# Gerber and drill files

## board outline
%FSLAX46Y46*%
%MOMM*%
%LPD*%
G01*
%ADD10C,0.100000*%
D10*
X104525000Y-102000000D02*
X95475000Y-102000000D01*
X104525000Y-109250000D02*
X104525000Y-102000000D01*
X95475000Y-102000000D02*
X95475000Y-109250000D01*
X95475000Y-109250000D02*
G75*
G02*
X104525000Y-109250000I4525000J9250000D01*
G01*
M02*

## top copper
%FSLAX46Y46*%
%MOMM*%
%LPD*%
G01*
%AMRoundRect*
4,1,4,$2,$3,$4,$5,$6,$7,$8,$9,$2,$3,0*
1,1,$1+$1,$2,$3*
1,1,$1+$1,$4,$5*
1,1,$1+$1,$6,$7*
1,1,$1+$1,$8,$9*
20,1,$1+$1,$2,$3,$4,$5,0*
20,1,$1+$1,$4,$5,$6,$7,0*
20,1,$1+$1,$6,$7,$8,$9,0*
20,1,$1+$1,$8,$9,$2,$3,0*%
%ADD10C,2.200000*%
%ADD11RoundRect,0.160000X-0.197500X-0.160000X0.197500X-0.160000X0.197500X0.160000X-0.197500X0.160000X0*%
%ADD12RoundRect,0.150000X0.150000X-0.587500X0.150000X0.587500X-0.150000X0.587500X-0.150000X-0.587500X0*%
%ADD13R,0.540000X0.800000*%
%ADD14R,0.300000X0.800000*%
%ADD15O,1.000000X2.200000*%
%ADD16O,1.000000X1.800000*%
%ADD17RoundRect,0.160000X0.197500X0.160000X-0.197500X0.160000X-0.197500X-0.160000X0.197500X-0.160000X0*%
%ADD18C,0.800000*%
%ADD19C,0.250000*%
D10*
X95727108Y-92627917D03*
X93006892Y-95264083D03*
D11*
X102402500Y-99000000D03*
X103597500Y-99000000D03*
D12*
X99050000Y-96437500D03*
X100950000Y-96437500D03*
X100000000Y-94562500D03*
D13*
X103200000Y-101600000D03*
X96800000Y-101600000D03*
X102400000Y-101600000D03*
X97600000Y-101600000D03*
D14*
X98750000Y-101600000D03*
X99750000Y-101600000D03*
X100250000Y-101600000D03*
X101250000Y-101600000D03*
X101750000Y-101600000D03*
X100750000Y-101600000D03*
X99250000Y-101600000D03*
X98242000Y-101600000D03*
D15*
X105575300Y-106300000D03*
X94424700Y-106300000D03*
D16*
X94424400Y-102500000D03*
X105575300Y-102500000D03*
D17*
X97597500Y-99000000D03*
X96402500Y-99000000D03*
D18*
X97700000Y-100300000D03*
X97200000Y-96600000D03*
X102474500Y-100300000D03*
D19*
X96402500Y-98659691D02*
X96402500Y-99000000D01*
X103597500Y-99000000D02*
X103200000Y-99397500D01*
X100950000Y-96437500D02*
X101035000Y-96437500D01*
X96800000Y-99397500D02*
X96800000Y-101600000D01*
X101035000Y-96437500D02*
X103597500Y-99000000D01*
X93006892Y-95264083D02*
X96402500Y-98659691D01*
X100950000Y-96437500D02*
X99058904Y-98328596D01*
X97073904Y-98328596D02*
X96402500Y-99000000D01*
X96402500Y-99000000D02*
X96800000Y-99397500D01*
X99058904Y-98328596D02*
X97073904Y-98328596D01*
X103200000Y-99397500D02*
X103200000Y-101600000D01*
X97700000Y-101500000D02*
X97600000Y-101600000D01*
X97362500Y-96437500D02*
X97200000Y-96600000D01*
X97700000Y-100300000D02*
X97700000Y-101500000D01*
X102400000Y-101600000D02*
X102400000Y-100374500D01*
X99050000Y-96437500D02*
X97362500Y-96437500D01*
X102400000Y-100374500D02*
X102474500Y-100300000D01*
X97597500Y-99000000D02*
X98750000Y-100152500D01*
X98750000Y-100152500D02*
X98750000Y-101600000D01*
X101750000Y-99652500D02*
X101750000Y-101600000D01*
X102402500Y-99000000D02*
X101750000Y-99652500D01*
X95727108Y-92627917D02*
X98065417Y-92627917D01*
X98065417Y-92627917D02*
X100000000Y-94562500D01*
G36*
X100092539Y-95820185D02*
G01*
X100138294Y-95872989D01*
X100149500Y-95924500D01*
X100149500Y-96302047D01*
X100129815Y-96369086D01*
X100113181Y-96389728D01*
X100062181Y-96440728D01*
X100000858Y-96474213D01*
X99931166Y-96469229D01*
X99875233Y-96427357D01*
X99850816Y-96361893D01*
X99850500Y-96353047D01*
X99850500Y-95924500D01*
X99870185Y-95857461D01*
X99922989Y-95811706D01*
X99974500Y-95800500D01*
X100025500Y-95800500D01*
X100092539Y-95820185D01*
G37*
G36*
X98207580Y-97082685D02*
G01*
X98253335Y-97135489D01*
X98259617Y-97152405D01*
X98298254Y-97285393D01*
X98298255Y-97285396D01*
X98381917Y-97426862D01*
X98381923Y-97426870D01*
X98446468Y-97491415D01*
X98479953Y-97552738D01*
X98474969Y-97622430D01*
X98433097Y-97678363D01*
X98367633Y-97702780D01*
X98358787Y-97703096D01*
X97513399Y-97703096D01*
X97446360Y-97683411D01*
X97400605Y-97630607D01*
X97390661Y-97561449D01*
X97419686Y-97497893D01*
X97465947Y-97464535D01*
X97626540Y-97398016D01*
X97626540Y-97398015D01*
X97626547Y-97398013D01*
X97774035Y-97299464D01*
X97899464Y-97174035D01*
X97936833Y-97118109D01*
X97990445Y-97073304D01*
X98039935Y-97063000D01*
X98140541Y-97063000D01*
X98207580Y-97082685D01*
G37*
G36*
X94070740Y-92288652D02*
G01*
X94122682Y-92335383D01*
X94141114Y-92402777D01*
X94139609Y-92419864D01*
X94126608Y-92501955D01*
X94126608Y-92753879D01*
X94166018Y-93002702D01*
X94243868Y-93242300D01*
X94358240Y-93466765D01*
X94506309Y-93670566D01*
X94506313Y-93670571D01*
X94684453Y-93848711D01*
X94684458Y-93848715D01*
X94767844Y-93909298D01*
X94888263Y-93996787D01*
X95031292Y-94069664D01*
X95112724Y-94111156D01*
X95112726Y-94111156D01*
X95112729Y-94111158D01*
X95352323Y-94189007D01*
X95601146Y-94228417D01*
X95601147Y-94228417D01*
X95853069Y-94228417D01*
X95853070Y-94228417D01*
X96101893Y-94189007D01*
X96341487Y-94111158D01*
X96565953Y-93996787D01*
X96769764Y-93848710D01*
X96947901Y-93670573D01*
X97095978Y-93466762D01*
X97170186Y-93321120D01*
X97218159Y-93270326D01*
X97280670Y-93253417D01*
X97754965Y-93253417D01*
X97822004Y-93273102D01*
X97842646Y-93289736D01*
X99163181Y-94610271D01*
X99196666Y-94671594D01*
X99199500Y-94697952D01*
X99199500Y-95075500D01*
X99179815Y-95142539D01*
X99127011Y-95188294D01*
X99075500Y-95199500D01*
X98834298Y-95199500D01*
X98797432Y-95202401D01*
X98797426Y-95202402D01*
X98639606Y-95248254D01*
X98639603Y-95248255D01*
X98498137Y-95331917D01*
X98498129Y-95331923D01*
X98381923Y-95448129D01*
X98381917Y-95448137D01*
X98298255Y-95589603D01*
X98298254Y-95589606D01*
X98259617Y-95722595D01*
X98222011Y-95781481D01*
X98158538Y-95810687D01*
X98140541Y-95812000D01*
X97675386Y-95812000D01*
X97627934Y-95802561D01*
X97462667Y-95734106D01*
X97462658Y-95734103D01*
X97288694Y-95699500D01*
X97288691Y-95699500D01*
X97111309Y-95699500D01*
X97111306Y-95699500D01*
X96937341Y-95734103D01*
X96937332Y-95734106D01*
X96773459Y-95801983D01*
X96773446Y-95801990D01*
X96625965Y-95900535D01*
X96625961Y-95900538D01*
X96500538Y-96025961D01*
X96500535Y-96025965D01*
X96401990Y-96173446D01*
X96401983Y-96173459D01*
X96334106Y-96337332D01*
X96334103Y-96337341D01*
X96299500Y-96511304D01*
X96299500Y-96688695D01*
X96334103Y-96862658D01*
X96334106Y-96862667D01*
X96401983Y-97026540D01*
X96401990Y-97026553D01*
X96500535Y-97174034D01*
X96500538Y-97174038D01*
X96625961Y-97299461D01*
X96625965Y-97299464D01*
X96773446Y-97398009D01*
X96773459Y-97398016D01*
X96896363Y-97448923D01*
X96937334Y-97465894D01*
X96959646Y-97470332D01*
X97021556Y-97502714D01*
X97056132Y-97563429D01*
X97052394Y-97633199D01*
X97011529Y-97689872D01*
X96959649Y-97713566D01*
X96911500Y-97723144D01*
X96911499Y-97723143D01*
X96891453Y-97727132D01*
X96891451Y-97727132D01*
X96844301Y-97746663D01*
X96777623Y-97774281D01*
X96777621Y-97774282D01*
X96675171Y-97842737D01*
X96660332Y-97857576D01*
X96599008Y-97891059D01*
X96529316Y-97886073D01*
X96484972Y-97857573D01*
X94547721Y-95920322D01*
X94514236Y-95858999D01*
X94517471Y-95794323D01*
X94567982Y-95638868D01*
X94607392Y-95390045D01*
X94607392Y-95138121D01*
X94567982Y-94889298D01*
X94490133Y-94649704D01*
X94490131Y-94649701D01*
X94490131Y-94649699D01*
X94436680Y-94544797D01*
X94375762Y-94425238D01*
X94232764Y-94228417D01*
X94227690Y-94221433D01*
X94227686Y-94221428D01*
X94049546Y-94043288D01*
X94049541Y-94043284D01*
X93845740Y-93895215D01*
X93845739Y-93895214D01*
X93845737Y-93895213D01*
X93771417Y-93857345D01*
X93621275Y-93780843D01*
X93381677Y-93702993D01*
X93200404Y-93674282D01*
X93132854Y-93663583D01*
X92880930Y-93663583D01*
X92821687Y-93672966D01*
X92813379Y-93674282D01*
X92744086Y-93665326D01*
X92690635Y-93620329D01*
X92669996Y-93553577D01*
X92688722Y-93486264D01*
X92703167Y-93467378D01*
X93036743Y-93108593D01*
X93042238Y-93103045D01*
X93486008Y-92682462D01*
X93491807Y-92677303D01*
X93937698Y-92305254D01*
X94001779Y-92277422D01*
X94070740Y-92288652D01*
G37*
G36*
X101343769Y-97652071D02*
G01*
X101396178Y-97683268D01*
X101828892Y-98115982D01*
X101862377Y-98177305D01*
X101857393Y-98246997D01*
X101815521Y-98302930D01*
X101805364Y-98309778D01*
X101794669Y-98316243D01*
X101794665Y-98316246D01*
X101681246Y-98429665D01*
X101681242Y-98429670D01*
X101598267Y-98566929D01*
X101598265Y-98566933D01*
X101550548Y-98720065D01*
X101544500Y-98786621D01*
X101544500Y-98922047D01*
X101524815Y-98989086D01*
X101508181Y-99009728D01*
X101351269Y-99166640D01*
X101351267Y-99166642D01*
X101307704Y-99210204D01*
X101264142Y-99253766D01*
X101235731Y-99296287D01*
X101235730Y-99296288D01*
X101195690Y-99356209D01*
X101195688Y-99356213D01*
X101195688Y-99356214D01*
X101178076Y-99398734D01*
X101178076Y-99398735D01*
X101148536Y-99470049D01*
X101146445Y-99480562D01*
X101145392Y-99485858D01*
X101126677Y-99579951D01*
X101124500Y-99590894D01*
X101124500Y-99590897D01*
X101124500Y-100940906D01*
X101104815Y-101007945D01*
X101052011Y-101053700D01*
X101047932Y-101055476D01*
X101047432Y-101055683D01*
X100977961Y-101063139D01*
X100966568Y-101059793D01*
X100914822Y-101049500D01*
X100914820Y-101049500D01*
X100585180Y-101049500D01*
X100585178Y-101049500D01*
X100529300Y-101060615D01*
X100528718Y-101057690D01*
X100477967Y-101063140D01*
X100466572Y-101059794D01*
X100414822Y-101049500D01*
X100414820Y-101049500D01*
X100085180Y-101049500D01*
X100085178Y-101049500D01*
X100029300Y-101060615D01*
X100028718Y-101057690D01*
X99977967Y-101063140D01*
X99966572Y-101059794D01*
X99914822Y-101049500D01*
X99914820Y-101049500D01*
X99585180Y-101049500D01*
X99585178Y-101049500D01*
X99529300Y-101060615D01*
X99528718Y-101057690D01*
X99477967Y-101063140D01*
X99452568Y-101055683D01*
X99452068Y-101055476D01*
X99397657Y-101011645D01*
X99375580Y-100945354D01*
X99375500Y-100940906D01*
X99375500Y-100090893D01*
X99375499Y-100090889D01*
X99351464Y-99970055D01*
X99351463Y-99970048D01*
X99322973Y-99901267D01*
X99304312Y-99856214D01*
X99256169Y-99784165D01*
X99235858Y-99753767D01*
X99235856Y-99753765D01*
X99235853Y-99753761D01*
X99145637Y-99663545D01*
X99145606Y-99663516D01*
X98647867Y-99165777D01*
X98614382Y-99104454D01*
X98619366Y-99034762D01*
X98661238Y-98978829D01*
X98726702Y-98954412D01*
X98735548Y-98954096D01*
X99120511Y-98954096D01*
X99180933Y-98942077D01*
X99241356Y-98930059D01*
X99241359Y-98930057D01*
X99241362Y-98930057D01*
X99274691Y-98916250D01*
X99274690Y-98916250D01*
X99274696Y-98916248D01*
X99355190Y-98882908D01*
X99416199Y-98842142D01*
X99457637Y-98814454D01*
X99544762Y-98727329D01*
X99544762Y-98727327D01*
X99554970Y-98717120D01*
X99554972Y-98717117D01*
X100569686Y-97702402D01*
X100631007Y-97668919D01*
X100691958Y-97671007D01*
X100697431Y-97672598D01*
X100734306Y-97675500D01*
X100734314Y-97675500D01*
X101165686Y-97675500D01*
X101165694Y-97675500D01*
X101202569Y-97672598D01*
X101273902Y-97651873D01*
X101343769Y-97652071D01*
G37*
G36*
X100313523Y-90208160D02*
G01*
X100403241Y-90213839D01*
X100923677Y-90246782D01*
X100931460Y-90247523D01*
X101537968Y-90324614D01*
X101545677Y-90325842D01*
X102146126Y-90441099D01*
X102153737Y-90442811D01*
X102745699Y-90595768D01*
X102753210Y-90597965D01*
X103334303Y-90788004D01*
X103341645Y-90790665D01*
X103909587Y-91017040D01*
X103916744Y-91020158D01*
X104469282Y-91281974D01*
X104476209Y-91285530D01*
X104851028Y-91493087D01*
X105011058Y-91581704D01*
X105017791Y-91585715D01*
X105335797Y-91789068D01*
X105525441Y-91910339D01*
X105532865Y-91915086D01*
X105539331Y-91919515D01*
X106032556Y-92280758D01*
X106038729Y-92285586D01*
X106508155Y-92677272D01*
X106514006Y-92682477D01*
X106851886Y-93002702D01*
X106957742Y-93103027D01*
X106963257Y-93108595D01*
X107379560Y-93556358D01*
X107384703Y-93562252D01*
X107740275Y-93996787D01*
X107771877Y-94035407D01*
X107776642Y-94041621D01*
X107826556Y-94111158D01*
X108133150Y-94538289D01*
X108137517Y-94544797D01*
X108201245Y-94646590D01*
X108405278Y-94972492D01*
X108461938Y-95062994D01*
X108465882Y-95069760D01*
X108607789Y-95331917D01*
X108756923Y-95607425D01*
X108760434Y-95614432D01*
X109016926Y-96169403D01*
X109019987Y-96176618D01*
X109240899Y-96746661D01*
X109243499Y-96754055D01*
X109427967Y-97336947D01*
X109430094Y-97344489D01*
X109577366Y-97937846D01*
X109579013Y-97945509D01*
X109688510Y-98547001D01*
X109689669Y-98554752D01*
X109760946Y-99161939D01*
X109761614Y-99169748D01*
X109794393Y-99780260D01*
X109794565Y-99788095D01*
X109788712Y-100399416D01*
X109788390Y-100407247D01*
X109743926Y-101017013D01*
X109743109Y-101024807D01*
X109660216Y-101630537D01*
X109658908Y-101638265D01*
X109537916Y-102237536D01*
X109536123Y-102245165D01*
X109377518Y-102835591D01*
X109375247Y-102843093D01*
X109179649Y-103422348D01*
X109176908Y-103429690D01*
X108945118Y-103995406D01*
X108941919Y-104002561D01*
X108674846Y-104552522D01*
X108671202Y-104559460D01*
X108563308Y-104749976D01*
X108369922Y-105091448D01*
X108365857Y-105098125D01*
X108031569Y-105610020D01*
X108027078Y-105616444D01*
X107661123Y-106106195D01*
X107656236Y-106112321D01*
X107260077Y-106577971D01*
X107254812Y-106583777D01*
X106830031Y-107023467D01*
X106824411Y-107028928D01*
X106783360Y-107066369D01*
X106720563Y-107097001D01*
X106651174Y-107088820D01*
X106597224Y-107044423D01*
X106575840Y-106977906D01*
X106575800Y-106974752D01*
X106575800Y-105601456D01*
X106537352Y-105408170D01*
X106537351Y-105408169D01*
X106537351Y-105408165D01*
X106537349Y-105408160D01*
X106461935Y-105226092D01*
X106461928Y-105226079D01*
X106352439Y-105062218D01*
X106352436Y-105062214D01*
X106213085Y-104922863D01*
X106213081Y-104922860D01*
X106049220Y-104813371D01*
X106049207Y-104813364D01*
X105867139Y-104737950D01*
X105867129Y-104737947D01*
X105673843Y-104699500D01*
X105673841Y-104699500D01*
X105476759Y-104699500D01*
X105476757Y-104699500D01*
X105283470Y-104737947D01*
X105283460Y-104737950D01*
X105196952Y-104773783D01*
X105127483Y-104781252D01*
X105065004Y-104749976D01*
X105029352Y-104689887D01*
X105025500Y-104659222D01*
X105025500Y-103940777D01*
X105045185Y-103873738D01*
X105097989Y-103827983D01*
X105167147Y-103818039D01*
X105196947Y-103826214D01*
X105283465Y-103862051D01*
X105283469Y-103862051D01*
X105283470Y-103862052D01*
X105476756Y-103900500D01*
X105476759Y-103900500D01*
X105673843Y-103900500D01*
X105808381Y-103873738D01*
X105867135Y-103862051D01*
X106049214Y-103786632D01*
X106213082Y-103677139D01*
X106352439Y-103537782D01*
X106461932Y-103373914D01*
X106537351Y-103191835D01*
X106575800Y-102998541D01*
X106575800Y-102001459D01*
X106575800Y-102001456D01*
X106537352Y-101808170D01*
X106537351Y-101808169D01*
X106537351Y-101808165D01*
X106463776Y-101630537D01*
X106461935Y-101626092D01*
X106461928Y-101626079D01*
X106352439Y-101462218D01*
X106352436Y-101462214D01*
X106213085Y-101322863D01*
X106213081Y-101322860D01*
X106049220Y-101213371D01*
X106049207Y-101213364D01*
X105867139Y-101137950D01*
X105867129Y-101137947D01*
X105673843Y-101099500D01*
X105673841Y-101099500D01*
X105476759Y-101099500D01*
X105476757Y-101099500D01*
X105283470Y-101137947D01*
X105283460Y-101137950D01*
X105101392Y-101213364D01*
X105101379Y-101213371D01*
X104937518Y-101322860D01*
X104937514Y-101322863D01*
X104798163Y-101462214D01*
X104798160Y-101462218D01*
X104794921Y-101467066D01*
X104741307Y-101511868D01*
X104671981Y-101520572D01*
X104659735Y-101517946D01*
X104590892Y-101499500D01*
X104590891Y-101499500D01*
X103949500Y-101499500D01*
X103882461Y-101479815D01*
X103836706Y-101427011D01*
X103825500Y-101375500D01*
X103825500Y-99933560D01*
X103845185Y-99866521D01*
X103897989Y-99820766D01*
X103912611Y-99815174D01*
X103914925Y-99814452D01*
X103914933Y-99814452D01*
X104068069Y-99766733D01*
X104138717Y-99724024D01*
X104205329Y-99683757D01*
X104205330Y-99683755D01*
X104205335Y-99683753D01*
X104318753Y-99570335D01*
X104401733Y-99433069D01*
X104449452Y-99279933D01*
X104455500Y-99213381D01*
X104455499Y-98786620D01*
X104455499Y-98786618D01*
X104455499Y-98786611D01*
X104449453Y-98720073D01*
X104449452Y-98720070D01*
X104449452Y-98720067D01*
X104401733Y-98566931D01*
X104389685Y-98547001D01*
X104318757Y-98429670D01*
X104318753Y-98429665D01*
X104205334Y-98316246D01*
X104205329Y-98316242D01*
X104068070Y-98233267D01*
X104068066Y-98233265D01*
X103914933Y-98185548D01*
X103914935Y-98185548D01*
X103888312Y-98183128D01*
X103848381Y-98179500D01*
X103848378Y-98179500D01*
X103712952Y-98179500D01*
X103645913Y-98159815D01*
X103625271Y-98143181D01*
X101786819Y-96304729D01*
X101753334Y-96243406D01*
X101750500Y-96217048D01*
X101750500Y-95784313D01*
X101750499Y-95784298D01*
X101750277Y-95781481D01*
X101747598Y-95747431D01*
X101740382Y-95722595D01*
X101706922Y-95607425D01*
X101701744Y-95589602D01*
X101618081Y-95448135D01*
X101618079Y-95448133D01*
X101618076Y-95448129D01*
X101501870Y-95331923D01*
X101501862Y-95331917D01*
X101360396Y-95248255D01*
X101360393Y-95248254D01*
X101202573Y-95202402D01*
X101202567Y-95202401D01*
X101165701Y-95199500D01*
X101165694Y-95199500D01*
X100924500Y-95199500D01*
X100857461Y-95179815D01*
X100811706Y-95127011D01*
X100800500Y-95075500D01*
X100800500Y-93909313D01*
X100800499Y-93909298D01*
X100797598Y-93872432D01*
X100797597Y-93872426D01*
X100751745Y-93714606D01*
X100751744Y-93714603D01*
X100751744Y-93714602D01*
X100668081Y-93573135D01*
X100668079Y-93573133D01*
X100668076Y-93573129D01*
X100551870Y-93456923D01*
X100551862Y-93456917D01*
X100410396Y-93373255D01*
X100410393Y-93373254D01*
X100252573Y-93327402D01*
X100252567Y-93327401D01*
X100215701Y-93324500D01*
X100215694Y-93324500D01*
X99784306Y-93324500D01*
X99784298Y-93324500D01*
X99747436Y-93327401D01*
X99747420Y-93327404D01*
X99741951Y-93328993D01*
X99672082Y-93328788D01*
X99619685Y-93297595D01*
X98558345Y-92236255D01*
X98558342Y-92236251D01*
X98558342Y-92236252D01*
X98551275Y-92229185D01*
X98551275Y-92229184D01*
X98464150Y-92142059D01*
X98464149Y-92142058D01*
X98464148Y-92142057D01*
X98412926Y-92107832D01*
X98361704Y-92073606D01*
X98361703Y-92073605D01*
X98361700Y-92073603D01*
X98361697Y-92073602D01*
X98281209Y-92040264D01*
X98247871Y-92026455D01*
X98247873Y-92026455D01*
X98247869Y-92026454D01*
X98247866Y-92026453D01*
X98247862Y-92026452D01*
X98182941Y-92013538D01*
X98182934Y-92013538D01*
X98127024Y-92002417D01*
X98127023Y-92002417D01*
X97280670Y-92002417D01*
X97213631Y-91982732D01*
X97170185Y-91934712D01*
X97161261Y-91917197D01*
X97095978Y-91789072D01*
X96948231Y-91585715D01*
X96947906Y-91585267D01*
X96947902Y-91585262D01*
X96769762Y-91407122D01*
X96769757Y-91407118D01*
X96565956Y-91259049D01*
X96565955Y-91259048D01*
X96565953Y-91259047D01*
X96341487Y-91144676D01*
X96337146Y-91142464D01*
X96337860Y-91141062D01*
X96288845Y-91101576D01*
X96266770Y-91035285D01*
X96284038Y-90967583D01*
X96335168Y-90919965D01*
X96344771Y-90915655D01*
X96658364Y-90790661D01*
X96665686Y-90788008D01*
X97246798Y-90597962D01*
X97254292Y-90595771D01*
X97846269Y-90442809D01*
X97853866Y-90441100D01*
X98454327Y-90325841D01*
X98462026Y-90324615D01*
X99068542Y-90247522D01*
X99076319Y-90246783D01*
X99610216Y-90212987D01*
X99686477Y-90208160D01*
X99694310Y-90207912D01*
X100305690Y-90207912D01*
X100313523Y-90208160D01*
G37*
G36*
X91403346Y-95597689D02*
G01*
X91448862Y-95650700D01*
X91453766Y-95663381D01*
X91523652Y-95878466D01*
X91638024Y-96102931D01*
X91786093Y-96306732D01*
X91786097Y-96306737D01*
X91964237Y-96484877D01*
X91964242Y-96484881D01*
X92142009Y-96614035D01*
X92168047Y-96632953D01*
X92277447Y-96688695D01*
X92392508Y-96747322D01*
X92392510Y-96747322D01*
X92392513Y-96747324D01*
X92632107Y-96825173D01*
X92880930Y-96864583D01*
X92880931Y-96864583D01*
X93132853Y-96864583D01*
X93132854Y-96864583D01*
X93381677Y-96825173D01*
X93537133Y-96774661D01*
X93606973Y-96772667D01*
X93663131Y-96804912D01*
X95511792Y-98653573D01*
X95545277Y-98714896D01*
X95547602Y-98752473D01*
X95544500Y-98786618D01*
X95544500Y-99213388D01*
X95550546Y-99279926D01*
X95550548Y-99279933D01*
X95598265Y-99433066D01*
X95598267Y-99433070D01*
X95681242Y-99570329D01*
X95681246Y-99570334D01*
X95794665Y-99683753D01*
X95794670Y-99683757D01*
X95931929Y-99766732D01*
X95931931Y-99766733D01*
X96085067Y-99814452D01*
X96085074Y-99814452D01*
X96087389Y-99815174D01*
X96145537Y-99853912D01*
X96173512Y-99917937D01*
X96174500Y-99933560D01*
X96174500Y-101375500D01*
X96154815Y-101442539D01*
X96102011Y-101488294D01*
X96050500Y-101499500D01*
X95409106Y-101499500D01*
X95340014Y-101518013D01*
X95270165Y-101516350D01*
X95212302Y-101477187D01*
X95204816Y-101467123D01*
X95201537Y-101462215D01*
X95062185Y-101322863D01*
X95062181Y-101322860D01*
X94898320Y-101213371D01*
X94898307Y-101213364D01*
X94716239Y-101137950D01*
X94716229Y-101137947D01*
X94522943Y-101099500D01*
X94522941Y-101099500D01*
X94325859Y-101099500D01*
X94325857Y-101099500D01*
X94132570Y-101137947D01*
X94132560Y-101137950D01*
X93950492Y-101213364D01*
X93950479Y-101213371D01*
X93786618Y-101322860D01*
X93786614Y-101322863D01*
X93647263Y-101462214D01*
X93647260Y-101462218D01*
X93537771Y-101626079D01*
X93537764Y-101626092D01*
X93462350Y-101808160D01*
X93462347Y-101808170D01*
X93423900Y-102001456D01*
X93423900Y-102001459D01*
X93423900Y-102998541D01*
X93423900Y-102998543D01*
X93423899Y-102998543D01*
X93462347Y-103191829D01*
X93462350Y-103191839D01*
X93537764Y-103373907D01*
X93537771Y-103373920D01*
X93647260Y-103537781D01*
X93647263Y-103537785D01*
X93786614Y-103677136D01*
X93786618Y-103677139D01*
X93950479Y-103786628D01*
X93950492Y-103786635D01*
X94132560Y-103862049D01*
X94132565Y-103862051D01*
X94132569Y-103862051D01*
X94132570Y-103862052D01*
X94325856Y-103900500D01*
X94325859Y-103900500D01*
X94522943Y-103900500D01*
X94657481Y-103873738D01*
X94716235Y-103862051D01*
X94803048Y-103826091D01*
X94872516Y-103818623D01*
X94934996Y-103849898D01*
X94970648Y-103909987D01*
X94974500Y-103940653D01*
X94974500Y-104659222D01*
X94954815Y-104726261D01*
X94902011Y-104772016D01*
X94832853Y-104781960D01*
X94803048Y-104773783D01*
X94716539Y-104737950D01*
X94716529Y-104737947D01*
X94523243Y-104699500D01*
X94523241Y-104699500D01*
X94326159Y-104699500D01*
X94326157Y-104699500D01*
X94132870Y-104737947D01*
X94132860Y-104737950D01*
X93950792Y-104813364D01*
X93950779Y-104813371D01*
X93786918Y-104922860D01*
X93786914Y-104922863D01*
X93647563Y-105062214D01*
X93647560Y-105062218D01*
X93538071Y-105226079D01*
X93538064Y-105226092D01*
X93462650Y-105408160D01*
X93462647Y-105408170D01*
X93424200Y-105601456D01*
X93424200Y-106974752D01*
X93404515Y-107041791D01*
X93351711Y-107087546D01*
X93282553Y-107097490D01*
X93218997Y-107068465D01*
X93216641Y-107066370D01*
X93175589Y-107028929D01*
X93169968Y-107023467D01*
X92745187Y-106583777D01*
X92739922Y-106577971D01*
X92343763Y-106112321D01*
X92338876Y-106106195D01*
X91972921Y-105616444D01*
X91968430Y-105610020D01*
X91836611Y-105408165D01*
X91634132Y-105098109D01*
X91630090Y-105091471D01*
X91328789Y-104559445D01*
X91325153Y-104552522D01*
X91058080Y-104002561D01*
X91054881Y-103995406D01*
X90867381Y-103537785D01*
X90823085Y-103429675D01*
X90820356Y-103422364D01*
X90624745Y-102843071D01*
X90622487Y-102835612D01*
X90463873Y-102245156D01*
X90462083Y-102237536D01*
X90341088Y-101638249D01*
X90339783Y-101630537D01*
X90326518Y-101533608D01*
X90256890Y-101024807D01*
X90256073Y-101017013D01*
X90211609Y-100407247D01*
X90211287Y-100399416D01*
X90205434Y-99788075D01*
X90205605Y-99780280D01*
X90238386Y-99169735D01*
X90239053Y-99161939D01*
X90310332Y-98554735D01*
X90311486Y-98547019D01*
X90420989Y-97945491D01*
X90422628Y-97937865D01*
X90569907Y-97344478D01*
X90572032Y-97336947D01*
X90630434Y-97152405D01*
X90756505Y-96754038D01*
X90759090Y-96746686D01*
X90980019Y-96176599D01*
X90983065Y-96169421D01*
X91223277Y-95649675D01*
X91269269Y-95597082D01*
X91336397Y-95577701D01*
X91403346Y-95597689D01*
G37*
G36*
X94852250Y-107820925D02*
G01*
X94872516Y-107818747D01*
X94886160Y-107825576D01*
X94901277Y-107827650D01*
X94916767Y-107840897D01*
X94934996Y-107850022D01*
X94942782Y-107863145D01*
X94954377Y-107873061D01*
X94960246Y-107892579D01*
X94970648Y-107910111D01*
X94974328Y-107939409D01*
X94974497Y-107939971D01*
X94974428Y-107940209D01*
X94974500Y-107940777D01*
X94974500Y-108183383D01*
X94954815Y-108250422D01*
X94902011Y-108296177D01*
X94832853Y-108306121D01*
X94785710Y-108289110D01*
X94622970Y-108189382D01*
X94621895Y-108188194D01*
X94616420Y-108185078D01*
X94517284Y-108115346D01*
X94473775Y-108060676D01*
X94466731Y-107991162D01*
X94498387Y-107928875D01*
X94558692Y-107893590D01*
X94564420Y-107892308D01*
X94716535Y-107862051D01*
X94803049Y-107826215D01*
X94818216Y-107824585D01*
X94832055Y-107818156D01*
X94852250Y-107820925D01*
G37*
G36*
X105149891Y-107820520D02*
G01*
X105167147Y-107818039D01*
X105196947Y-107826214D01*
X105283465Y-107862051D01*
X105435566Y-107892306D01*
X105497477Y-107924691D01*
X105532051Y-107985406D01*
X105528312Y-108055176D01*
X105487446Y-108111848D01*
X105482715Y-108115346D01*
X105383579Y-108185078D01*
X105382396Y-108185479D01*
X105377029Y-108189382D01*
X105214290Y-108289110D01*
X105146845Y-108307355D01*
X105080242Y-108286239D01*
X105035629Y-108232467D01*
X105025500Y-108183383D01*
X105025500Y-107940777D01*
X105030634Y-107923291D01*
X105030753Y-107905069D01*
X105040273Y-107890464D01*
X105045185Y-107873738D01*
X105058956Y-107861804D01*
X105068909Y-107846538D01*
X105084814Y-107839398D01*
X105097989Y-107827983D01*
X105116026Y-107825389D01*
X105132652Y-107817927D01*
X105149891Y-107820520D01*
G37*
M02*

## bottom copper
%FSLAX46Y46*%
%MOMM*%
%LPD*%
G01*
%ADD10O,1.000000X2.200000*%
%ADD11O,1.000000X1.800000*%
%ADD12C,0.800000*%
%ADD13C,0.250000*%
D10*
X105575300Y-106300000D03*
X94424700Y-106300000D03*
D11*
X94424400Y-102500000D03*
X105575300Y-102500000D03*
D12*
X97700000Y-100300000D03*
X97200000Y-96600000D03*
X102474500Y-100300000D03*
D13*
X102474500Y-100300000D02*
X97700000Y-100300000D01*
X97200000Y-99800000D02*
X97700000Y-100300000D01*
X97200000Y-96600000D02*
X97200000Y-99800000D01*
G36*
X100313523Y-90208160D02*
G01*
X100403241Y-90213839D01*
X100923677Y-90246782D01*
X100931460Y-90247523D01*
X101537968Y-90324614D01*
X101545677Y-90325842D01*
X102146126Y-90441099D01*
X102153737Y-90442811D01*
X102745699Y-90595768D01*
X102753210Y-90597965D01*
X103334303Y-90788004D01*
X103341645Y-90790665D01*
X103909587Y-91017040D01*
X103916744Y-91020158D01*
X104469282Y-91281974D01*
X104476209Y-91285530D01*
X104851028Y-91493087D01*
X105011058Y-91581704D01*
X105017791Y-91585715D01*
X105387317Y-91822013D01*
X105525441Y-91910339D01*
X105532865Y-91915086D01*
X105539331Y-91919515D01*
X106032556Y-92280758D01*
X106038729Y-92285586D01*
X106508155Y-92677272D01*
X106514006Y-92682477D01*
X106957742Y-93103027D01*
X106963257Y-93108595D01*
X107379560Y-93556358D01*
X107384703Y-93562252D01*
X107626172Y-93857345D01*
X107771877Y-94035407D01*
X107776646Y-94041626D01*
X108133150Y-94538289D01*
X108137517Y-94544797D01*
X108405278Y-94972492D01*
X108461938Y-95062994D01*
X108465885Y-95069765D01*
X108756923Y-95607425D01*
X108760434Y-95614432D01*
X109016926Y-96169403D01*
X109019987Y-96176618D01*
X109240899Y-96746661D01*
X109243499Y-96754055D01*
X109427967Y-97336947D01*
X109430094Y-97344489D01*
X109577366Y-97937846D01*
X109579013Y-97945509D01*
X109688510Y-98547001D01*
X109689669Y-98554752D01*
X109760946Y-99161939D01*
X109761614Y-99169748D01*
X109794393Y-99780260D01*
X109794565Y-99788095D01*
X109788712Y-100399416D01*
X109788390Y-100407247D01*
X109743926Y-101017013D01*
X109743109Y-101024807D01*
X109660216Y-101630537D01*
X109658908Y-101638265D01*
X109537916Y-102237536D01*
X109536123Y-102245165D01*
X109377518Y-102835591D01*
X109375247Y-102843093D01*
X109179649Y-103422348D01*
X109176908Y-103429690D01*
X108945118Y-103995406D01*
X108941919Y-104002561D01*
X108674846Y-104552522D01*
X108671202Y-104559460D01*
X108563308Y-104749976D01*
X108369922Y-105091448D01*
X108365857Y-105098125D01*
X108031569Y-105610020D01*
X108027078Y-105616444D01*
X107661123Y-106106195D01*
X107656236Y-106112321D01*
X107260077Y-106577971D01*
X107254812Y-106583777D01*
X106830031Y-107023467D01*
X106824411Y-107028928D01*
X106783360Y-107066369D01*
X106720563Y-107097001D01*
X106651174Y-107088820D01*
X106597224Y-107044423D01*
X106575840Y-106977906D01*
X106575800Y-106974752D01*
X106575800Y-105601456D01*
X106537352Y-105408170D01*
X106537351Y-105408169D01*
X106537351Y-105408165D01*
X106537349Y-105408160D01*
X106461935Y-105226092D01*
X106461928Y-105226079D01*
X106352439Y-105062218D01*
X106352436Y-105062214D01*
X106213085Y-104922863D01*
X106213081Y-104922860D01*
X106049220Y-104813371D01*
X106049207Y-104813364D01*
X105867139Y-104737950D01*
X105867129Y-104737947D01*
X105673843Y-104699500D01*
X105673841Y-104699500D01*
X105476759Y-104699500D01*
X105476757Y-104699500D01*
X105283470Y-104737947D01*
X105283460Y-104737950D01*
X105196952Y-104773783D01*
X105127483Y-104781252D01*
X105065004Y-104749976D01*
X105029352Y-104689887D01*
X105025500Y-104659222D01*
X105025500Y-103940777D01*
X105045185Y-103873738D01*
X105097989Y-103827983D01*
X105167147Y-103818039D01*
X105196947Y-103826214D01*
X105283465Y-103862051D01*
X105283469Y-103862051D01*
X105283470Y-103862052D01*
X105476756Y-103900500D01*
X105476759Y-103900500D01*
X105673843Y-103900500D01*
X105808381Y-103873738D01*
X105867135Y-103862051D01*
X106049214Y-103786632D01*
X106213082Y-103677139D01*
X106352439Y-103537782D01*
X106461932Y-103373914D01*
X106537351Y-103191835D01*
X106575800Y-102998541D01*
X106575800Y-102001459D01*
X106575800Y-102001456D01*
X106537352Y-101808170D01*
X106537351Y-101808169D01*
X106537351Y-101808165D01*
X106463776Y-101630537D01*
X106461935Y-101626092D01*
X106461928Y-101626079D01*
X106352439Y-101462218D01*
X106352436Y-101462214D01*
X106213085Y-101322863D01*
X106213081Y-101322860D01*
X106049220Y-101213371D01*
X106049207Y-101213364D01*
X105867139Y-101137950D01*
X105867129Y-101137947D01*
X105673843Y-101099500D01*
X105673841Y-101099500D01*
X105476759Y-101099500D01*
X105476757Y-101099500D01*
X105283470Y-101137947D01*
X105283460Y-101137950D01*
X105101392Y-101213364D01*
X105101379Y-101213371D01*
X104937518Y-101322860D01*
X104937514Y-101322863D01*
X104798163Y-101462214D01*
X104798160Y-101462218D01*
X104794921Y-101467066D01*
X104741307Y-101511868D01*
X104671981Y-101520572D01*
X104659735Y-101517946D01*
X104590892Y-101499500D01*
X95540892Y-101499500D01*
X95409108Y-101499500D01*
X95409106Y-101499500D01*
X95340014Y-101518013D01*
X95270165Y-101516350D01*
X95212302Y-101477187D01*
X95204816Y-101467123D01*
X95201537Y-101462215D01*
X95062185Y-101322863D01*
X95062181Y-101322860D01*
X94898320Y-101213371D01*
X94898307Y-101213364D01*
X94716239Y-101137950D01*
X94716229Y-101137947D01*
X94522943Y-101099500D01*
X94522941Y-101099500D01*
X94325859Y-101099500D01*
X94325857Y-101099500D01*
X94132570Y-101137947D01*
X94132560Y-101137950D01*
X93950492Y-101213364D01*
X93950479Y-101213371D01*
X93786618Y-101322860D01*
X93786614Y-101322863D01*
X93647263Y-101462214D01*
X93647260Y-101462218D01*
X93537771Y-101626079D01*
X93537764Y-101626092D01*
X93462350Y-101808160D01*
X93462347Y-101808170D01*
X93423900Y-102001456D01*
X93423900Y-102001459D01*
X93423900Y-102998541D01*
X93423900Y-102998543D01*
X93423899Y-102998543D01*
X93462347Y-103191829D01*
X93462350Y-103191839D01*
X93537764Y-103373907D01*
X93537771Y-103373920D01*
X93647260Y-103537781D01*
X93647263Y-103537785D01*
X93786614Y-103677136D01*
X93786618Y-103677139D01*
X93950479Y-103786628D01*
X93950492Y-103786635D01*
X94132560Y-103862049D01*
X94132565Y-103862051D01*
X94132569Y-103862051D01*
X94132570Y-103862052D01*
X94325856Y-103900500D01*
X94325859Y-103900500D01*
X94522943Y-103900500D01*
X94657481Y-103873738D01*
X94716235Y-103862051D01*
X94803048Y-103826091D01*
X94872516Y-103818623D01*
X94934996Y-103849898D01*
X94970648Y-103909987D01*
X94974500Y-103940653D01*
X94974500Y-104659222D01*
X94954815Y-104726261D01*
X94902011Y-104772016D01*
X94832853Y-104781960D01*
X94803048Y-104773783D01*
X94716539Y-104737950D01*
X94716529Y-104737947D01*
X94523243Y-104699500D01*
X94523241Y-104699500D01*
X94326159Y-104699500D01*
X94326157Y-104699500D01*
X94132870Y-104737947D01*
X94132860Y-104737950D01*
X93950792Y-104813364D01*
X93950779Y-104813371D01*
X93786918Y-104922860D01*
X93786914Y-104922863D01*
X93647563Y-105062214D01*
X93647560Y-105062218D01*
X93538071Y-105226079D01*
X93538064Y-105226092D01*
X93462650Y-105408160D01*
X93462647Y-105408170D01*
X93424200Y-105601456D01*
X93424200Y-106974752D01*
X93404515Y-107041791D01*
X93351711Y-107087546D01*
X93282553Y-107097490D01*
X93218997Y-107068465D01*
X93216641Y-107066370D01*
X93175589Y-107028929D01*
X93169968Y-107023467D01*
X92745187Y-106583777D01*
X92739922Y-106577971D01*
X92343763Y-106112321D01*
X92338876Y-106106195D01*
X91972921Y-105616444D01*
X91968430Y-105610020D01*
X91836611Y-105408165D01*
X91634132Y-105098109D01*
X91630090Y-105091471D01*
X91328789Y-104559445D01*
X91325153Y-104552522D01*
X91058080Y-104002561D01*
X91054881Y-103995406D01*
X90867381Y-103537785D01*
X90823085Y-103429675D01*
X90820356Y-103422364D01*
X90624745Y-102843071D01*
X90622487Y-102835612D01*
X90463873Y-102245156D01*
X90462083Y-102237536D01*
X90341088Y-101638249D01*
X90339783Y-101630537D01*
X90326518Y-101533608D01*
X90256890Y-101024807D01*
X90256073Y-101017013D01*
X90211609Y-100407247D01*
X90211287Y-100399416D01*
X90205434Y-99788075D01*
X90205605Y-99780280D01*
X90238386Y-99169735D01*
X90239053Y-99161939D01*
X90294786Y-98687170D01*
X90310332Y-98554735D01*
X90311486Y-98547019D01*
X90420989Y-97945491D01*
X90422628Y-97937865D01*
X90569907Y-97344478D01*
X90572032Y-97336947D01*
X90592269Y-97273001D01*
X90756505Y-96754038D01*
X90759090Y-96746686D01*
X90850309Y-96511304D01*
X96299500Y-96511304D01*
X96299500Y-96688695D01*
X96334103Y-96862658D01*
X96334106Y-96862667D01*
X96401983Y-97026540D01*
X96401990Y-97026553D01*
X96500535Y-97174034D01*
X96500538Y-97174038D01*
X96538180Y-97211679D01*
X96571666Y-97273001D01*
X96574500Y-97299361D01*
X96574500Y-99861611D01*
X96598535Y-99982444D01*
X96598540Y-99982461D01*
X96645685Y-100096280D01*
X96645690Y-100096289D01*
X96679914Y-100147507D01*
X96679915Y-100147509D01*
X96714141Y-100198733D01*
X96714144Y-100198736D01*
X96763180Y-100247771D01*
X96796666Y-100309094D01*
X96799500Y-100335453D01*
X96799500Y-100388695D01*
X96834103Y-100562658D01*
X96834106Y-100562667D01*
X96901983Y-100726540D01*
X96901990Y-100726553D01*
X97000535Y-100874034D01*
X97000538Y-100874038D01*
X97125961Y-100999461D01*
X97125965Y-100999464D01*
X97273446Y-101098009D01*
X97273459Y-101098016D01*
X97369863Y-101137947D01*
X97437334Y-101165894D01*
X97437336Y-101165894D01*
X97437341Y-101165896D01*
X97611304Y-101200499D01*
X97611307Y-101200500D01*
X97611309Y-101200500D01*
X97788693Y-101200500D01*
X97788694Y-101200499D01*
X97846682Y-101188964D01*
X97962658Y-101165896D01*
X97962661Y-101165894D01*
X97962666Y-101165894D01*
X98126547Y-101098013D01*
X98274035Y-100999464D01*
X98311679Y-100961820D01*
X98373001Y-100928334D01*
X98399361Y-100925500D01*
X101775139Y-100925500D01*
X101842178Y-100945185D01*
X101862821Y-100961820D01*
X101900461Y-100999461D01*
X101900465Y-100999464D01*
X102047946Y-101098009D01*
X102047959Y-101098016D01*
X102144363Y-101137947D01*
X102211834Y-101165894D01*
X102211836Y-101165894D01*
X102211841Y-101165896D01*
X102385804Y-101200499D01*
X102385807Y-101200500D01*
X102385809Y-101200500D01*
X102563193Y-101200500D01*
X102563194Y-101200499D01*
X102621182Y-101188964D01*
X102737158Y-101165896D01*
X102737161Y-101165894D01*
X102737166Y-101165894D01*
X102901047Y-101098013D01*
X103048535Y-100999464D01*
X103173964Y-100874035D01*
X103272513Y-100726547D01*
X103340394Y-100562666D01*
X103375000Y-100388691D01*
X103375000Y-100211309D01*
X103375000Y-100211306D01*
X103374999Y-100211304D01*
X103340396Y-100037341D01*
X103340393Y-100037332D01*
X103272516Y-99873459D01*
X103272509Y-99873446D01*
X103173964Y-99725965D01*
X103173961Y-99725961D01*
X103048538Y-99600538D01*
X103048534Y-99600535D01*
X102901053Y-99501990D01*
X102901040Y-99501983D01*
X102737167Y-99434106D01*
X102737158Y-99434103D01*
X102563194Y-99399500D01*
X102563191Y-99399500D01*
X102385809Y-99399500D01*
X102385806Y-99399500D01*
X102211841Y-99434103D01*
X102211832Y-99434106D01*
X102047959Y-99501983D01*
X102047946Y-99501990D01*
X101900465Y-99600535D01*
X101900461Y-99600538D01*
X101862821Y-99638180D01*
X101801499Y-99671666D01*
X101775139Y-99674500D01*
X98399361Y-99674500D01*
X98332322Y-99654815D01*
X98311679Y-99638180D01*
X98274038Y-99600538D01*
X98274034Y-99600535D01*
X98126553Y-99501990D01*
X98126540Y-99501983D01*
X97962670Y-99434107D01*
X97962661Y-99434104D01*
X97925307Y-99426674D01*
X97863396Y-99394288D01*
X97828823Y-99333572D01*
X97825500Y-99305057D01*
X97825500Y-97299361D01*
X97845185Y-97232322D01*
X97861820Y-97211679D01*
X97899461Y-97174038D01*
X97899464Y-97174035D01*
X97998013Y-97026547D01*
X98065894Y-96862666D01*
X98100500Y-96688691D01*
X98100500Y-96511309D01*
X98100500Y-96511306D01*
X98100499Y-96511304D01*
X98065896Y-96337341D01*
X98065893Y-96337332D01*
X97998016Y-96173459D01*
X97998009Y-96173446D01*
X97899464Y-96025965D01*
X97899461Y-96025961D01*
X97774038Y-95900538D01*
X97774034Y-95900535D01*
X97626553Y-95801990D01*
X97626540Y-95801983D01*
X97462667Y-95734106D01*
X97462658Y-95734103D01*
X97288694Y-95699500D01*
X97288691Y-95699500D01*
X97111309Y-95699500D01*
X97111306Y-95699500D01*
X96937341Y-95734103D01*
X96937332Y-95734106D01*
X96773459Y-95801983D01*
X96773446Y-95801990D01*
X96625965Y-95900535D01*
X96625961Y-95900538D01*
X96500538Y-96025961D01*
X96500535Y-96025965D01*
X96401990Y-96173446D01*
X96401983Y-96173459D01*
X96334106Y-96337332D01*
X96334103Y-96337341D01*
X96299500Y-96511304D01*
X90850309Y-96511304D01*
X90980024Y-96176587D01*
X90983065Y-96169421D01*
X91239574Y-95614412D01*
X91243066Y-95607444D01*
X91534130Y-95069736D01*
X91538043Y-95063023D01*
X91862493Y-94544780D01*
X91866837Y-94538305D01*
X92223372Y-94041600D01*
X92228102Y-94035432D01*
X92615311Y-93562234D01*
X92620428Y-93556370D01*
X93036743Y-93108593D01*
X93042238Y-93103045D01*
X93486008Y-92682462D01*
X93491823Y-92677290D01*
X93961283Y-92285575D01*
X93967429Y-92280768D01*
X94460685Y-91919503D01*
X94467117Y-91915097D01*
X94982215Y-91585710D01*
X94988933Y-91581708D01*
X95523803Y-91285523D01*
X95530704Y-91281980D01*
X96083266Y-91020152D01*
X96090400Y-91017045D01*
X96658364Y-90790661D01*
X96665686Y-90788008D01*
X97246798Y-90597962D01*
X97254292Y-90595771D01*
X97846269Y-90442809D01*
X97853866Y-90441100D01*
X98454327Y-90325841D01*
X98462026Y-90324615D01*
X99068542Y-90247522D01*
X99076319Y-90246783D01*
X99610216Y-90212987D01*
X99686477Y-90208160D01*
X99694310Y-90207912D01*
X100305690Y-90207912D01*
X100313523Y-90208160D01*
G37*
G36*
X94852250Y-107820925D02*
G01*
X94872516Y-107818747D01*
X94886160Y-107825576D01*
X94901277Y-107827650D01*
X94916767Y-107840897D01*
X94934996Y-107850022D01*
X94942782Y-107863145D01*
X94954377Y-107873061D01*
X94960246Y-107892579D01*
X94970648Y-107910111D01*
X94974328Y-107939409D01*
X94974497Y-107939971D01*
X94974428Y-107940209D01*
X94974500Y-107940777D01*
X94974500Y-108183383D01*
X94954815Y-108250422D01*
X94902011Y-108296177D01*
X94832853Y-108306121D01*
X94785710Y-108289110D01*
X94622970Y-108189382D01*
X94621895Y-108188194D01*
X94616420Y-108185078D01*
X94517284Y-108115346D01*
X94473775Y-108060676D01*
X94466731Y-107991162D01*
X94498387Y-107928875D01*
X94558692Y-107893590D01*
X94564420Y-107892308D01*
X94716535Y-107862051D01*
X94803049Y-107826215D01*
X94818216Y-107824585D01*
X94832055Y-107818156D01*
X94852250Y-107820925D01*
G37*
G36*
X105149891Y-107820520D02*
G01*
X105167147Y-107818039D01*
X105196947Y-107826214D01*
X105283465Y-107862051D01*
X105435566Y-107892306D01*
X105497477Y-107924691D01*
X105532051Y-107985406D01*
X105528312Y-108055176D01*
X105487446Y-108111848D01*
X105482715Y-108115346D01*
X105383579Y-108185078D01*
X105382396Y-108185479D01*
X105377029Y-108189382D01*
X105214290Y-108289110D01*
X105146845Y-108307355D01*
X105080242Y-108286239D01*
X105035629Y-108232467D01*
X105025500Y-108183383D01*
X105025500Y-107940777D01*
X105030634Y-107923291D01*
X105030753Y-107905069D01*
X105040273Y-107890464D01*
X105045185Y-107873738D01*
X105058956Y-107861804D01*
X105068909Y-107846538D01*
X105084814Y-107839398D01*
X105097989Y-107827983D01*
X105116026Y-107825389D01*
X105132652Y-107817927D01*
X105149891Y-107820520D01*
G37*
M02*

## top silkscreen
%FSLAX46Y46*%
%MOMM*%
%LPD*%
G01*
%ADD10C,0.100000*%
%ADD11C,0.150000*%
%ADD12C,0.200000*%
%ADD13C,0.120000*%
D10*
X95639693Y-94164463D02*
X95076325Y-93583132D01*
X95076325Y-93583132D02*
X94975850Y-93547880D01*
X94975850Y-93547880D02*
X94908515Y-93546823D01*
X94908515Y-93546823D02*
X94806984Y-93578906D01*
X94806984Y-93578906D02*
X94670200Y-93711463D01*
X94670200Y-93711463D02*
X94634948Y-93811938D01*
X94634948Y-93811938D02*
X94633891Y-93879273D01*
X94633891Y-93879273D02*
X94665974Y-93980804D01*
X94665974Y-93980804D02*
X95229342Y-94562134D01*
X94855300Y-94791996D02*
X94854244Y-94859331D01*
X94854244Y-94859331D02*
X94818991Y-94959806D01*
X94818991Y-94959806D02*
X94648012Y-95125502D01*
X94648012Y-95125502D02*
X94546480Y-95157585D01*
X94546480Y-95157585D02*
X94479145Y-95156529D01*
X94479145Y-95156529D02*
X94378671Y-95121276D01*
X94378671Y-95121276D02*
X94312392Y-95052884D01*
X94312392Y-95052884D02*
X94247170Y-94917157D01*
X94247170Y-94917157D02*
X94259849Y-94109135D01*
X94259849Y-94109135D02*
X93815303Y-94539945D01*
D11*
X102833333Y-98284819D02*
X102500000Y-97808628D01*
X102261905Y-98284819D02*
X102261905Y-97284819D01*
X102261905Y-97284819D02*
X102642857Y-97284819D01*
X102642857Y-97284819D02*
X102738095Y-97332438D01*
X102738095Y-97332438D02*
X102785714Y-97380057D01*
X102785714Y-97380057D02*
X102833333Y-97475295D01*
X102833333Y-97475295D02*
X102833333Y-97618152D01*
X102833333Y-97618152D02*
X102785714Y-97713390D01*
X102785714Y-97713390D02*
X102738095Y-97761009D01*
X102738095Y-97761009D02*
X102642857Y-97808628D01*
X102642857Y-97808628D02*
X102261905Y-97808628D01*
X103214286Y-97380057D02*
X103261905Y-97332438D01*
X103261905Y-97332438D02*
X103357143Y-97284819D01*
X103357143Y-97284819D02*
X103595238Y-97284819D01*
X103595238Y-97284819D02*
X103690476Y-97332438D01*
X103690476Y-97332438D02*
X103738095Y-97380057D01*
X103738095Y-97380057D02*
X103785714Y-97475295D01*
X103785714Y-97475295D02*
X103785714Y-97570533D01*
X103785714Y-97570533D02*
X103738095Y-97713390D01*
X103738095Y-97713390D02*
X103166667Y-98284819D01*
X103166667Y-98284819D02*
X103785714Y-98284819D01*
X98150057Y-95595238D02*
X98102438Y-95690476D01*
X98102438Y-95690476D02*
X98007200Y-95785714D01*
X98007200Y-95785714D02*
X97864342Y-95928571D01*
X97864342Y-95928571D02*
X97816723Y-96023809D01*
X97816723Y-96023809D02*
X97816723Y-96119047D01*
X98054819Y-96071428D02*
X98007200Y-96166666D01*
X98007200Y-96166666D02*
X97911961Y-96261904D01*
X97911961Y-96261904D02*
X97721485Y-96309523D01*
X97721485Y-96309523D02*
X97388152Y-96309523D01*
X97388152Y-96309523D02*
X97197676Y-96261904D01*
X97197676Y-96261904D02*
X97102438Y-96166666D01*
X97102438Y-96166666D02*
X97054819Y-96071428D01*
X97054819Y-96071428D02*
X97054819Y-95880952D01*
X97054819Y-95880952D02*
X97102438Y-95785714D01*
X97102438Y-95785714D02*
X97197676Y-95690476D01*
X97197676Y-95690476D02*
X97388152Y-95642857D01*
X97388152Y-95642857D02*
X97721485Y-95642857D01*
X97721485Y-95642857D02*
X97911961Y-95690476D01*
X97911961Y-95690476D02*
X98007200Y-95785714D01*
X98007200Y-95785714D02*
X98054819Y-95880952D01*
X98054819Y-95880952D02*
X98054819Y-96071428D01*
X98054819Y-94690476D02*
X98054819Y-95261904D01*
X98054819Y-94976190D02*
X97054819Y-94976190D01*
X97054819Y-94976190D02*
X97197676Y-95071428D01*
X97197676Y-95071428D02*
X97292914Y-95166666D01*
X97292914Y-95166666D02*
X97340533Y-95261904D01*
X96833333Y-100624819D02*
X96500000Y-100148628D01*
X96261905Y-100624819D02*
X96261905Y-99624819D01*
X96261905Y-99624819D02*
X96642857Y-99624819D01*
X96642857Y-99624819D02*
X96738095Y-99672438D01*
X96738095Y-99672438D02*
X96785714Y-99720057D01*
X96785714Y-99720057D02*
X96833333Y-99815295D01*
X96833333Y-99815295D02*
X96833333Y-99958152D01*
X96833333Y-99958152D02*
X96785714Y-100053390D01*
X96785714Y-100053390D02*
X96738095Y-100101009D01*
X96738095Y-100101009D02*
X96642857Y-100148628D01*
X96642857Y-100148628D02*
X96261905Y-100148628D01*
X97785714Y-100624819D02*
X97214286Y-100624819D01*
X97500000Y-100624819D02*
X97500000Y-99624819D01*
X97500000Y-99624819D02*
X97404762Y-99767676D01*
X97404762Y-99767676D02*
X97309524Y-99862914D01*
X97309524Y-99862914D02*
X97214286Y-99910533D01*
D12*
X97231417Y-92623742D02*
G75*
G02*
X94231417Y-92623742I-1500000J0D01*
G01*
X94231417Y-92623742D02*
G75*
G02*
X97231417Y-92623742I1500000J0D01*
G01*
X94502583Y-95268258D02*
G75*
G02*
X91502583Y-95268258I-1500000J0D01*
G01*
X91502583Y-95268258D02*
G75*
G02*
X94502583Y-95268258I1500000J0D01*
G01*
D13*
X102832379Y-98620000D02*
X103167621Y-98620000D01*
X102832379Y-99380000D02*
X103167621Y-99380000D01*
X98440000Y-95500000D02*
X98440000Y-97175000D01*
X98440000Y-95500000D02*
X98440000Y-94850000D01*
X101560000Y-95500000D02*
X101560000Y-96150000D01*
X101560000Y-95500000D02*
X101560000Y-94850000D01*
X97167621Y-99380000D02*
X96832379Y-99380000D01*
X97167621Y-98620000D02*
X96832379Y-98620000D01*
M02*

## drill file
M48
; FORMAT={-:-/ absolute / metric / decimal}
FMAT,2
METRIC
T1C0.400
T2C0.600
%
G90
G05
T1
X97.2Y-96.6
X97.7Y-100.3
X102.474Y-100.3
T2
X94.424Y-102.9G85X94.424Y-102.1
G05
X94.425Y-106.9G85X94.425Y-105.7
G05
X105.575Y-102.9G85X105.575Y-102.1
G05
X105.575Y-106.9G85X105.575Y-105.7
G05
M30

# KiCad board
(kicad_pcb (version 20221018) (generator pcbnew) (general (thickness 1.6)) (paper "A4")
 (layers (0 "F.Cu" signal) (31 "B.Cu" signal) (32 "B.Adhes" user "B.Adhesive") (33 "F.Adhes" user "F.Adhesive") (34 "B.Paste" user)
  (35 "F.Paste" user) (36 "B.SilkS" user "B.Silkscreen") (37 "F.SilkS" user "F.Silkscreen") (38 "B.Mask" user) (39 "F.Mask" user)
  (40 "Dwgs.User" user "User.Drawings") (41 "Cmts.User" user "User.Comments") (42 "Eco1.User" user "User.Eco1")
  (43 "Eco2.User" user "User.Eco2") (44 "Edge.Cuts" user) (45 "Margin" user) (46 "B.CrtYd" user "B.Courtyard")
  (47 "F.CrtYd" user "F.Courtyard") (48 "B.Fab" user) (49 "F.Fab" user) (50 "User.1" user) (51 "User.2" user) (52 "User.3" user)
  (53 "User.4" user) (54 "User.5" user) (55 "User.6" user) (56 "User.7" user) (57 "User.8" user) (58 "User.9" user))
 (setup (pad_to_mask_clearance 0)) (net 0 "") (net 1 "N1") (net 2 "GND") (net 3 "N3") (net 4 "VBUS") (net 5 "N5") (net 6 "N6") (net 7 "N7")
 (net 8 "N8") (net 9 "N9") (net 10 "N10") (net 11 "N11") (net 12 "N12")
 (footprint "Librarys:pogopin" (layer "F.Cu") (at 94.367 93.946 -135.899)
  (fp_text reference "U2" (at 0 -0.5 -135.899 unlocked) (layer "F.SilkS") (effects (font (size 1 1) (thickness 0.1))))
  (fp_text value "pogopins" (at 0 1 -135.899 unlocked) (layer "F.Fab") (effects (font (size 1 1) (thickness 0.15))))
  (fp_circle (center -1.9 0) (end -0.4 0) (stroke (width 0.2) (type default)) (fill none) (layer "F.SilkS"))
  (fp_circle (center 1.9 0) (end 3.4 0) (stroke (width 0.2) (type default)) (fill none) (layer "F.SilkS"))
  (pad "1" smd circle (at -1.894 0 224.101) (size 2.2 2.2) (layers "F.Cu" "F.Paste" "F.Mask") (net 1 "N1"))
  (pad "2" smd circle (at 1.894 0 224.101) (size 2.2 2.2) (layers "F.Cu" "F.Paste" "F.Mask") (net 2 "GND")))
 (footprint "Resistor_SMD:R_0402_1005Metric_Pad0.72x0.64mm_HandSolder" (layer "F.Cu") (at 103 99)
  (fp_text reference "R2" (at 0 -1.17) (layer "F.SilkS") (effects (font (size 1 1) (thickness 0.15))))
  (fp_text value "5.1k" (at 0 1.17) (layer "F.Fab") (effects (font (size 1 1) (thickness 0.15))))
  (fp_line (start -0.167621 -0.38) (end 0.167621 -0.38) (stroke (width 0.12) (type solid)) (layer "F.SilkS"))
  (fp_line (start -0.167621 0.38) (end 0.167621 0.38) (stroke (width 0.12) (type solid)) (layer "F.SilkS"))
  (pad "1" smd roundrect (at -0.5975 0) (size 0.715 0.64) (layers "F.Cu" "F.Paste" "F.Mask") (roundrect_rratio 0.25) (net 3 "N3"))
  (pad "2" smd roundrect (at 0.5975 0) (size 0.715 0.64) (layers "F.Cu" "F.Paste" "F.Mask") (roundrect_rratio 0.25) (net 2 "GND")))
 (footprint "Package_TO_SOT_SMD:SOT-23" (layer "F.Cu") (at 100 95.5 90)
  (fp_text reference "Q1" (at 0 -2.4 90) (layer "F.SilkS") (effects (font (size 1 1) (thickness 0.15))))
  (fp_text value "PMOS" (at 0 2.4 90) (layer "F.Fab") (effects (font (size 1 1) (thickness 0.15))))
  (fp_line (start 0 -1.56) (end -1.675 -1.56) (stroke (width 0.12) (type solid)) (layer "F.SilkS"))
  (fp_line (start 0 -1.56) (end 0.65 -1.56) (stroke (width 0.12) (type solid)) (layer "F.SilkS"))
  (fp_line (start 0 1.56) (end -0.65 1.56) (stroke (width 0.12) (type solid)) (layer "F.SilkS"))
  (fp_line (start 0 1.56) (end 0.65 1.56) (stroke (width 0.12) (type solid)) (layer "F.SilkS"))
  (pad "1" smd roundrect (at -0.9375 -0.95 90) (size 1.475 0.6) (layers "F.Cu" "F.Paste" "F.Mask") (roundrect_rratio 0.25) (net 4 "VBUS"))
  (pad "2" smd roundrect (at -0.9375 0.95 90) (size 1.475 0.6) (layers "F.Cu" "F.Paste" "F.Mask") (roundrect_rratio 0.25) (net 2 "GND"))
  (pad "3" smd roundrect (at 0.9375 0 90) (size 1.475 0.6) (layers "F.Cu" "F.Paste" "F.Mask") (roundrect_rratio 0.25) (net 1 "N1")))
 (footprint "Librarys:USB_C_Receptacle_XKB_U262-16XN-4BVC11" (layer "F.Cu") (at 100 104.1 180)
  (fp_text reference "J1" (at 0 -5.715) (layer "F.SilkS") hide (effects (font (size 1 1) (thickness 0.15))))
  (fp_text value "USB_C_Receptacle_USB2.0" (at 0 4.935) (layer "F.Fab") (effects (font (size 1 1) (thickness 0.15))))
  (pad "A1" smd rect (at -3.2 2.5 180) (size 0.54 0.8) (layers "F.Cu" "F.Paste" "F.Mask") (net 2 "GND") (clearance 0.15))
  (pad "A1" smd rect (at 3.2 2.5 180) (size 0.54 0.8) (layers "F.Cu" "F.Paste" "F.Mask") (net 2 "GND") (clearance 0.15))
  (pad "A4" smd rect (at -2.4 2.5 180) (size 0.54 0.8) (layers "F.Cu" "F.Paste" "F.Mask") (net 4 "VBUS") (clearance 0.15))
  (pad "A4" smd rect (at 2.4 2.5 180) (size 0.54 0.8) (layers "F.Cu" "F.Paste" "F.Mask") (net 4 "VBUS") (clearance 0.15))
  (pad "A5" smd rect (at 1.25 2.5 180) (size 0.3 0.8) (layers "F.Cu" "F.Paste" "F.Mask") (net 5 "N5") (clearance 0.15))
  (pad "A6" smd rect (at 0.25 2.5 180) (size 0.3 0.8) (layers "F.Cu" "F.Paste" "F.Mask") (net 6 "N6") (clearance 0.15))
  (pad "A7" smd rect (at -0.25 2.5 180) (size 0.3 0.8) (layers "F.Cu" "F.Paste" "F.Mask") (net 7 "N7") (clearance 0.15))
  (pad "A8" smd rect (at -1.25 2.5 180) (size 0.3 0.8) (layers "F.Cu" "F.Paste" "F.Mask") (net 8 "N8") (clearance 0.15))
  (pad "B5" smd rect (at -1.75 2.5 180) (size 0.3 0.8) (layers "F.Cu" "F.Paste" "F.Mask") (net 3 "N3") (clearance 0.15))
  (pad "B6" smd rect (at -0.75 2.5 180) (size 0.3 0.8) (layers "F.Cu" "F.Paste" "F.Mask") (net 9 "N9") (clearance 0.15))
  (pad "B7" smd rect (at 0.75 2.5 180) (size 0.3 0.8) (layers "F.Cu" "F.Paste" "F.Mask") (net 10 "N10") (clearance 0.15))
  (pad "B8" smd rect (at 1.758 2.5 180) (size 0.3 0.8) (layers "F.Cu" "F.Paste" "F.Mask") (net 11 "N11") (clearance 0.15))
  (pad "S1" thru_hole oval (at -5.5753 -2.2 180) (size 1 2.2) (drill oval 0.6 1.8) (layers "*.Cu" "*.Mask") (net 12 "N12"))
  (pad "S2" thru_hole oval (at 5.5753 -2.2 180) (size 1 2.2) (drill oval 0.6 1.8) (layers "*.Cu" "*.Mask"))
  (pad "S3" thru_hole oval (at 5.5756 1.6 180) (size 1 1.8) (drill oval 0.6 1.4) (layers "*.Cu" "*.Mask"))
  (pad "S4" thru_hole oval (at -5.5753 1.6 180) (size 1 1.8) (drill oval 0.6 1.4) (layers "*.Cu" "*.Mask")))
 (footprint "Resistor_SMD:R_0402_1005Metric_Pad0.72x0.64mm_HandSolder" (layer "F.Cu") (at 97 99 180)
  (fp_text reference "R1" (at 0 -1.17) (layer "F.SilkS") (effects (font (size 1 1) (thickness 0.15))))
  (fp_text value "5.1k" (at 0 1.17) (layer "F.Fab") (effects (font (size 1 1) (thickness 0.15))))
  (fp_line (start -0.167621 -0.38) (end 0.167621 -0.38) (stroke (width 0.12) (type solid)) (layer "F.SilkS"))
  (fp_line (start -0.167621 0.38) (end 0.167621 0.38) (stroke (width 0.12) (type solid)) (layer "F.SilkS"))
  (pad "1" smd roundrect (at -0.5975 0 180) (size 0.715 0.64) (layers "F.Cu" "F.Paste" "F.Mask") (roundrect_rratio 0.25) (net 5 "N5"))
  (pad "2" smd roundrect (at 0.5975 0 180) (size 0.715 0.64) (layers "F.Cu" "F.Paste" "F.Mask") (roundrect_rratio 0.25) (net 2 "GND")))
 (gr_line (start 104.525 102) (end 95.475 102) (stroke (width 0.1) (type default)) (layer "Edge.Cuts"))
 (gr_line (start 104.525 109.25) (end 104.525 102) (stroke (width 0.1) (type default)) (layer "Edge.Cuts"))
 (gr_line (start 95.475 102) (end 95.475 109.25) (stroke (width 0.1) (type default)) (layer "Edge.Cuts"))
 (gr_arc (start 95.475 109.25) (mid 100 89.702519) (end 104.525 109.25) (stroke (width 0.1) (type default)) (layer "Edge.Cuts"))
 (segment (start 96.4025 98.659691) (end 96.4025 99) (width 0.25) (layer "F.Cu") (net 2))
 (segment (start 103.5975 99) (end 103.2 99.3975) (width 0.25) (layer "F.Cu") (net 2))
 (segment (start 100.95 96.4375) (end 101.035 96.4375) (width 0.25) (layer "F.Cu") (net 2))
 (segment (start 96.8 99.3975) (end 96.8 101.6) (width 0.25) (layer "F.Cu") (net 2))
 (segment (start 101.035 96.4375) (end 103.5975 99) (width 0.25) (layer "F.Cu") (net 2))
 (segment (start 93.006892 95.264083) (end 96.4025 98.659691) (width 0.25) (layer "F.Cu") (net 2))
 (segment (start 100.95 96.4375) (end 99.058904 98.328596) (width 0.25) (layer "F.Cu") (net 2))
 (segment (start 97.073904 98.328596) (end 96.4025 99) (width 0.25) (layer "F.Cu") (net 2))
 (segment (start 96.4025 99) (end 96.8 99.3975) (width 0.25) (layer "F.Cu") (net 2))
 (segment (start 99.058904 98.328596) (end 97.073904 98.328596) (width 0.25) (layer "F.Cu") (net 2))
 (segment (start 103.2 99.3975) (end 103.2 101.6) (width 0.25) (layer "F.Cu") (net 2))
 (segment (start 97.7 101.5) (end 97.6 101.6) (width 0.25) (layer "F.Cu") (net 4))
 (segment (start 97.3625 96.4375) (end 97.2 96.6) (width 0.25) (layer "F.Cu") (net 4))
 (segment (start 97.7 100.3) (end 97.7 101.5) (width 0.25) (layer "F.Cu") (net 4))
 (segment (start 102.4 101.6) (end 102.4 100.3745) (width 0.25) (layer "F.Cu") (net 4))
 (segment (start 99.05 96.4375) (end 97.3625 96.4375) (width 0.25) (layer "F.Cu") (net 4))
 (segment (start 102.4 100.3745) (end 102.4745 100.3) (width 0.25) (layer "F.Cu") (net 4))
 (via (at 97.7 100.3) (size 0.8) (drill 0.4) (layers "F.Cu" "B.Cu") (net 4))
 (via (at 97.2 96.6) (size 0.8) (drill 0.4) (layers "F.Cu" "B.Cu") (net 4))
 (via (at 102.4745 100.3) (size 0.8) (drill 0.4) (layers "F.Cu" "B.Cu") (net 4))
 (segment (start 102.4745 100.3) (end 97.7 100.3) (width 0.25) (layer "B.Cu") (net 4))
 (segment (start 97.2 99.8) (end 97.7 100.3) (width 0.25) (layer "B.Cu") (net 4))
 (segment (start 97.2 96.6) (end 97.2 99.8) (width 0.25) (layer "B.Cu") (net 4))
 (segment (start 97.5975 99) (end 98.75 100.1525) (width 0.25) (layer "F.Cu") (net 5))
 (segment (start 98.75 100.1525) (end 98.75 101.6) (width 0.25) (layer "F.Cu") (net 5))
 (segment (start 101.75 99.6525) (end 101.75 101.6) (width 0.25) (layer "F.Cu") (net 3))
 (segment (start 102.4025 99) (end 101.75 99.6525) (width 0.25) (layer "F.Cu") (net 3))
 (segment (start 95.727108 92.627917) (end 98.065417 92.627917) (width 0.25) (layer "F.Cu") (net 1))
 (segment (start 98.065417 92.627917) (end 100 94.5625) (width 0.25) (layer "F.Cu") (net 1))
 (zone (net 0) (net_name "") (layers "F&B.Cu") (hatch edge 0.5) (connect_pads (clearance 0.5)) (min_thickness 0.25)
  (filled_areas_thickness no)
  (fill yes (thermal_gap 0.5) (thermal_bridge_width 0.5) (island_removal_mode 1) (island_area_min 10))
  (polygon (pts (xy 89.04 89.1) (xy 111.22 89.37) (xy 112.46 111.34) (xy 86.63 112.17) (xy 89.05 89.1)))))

